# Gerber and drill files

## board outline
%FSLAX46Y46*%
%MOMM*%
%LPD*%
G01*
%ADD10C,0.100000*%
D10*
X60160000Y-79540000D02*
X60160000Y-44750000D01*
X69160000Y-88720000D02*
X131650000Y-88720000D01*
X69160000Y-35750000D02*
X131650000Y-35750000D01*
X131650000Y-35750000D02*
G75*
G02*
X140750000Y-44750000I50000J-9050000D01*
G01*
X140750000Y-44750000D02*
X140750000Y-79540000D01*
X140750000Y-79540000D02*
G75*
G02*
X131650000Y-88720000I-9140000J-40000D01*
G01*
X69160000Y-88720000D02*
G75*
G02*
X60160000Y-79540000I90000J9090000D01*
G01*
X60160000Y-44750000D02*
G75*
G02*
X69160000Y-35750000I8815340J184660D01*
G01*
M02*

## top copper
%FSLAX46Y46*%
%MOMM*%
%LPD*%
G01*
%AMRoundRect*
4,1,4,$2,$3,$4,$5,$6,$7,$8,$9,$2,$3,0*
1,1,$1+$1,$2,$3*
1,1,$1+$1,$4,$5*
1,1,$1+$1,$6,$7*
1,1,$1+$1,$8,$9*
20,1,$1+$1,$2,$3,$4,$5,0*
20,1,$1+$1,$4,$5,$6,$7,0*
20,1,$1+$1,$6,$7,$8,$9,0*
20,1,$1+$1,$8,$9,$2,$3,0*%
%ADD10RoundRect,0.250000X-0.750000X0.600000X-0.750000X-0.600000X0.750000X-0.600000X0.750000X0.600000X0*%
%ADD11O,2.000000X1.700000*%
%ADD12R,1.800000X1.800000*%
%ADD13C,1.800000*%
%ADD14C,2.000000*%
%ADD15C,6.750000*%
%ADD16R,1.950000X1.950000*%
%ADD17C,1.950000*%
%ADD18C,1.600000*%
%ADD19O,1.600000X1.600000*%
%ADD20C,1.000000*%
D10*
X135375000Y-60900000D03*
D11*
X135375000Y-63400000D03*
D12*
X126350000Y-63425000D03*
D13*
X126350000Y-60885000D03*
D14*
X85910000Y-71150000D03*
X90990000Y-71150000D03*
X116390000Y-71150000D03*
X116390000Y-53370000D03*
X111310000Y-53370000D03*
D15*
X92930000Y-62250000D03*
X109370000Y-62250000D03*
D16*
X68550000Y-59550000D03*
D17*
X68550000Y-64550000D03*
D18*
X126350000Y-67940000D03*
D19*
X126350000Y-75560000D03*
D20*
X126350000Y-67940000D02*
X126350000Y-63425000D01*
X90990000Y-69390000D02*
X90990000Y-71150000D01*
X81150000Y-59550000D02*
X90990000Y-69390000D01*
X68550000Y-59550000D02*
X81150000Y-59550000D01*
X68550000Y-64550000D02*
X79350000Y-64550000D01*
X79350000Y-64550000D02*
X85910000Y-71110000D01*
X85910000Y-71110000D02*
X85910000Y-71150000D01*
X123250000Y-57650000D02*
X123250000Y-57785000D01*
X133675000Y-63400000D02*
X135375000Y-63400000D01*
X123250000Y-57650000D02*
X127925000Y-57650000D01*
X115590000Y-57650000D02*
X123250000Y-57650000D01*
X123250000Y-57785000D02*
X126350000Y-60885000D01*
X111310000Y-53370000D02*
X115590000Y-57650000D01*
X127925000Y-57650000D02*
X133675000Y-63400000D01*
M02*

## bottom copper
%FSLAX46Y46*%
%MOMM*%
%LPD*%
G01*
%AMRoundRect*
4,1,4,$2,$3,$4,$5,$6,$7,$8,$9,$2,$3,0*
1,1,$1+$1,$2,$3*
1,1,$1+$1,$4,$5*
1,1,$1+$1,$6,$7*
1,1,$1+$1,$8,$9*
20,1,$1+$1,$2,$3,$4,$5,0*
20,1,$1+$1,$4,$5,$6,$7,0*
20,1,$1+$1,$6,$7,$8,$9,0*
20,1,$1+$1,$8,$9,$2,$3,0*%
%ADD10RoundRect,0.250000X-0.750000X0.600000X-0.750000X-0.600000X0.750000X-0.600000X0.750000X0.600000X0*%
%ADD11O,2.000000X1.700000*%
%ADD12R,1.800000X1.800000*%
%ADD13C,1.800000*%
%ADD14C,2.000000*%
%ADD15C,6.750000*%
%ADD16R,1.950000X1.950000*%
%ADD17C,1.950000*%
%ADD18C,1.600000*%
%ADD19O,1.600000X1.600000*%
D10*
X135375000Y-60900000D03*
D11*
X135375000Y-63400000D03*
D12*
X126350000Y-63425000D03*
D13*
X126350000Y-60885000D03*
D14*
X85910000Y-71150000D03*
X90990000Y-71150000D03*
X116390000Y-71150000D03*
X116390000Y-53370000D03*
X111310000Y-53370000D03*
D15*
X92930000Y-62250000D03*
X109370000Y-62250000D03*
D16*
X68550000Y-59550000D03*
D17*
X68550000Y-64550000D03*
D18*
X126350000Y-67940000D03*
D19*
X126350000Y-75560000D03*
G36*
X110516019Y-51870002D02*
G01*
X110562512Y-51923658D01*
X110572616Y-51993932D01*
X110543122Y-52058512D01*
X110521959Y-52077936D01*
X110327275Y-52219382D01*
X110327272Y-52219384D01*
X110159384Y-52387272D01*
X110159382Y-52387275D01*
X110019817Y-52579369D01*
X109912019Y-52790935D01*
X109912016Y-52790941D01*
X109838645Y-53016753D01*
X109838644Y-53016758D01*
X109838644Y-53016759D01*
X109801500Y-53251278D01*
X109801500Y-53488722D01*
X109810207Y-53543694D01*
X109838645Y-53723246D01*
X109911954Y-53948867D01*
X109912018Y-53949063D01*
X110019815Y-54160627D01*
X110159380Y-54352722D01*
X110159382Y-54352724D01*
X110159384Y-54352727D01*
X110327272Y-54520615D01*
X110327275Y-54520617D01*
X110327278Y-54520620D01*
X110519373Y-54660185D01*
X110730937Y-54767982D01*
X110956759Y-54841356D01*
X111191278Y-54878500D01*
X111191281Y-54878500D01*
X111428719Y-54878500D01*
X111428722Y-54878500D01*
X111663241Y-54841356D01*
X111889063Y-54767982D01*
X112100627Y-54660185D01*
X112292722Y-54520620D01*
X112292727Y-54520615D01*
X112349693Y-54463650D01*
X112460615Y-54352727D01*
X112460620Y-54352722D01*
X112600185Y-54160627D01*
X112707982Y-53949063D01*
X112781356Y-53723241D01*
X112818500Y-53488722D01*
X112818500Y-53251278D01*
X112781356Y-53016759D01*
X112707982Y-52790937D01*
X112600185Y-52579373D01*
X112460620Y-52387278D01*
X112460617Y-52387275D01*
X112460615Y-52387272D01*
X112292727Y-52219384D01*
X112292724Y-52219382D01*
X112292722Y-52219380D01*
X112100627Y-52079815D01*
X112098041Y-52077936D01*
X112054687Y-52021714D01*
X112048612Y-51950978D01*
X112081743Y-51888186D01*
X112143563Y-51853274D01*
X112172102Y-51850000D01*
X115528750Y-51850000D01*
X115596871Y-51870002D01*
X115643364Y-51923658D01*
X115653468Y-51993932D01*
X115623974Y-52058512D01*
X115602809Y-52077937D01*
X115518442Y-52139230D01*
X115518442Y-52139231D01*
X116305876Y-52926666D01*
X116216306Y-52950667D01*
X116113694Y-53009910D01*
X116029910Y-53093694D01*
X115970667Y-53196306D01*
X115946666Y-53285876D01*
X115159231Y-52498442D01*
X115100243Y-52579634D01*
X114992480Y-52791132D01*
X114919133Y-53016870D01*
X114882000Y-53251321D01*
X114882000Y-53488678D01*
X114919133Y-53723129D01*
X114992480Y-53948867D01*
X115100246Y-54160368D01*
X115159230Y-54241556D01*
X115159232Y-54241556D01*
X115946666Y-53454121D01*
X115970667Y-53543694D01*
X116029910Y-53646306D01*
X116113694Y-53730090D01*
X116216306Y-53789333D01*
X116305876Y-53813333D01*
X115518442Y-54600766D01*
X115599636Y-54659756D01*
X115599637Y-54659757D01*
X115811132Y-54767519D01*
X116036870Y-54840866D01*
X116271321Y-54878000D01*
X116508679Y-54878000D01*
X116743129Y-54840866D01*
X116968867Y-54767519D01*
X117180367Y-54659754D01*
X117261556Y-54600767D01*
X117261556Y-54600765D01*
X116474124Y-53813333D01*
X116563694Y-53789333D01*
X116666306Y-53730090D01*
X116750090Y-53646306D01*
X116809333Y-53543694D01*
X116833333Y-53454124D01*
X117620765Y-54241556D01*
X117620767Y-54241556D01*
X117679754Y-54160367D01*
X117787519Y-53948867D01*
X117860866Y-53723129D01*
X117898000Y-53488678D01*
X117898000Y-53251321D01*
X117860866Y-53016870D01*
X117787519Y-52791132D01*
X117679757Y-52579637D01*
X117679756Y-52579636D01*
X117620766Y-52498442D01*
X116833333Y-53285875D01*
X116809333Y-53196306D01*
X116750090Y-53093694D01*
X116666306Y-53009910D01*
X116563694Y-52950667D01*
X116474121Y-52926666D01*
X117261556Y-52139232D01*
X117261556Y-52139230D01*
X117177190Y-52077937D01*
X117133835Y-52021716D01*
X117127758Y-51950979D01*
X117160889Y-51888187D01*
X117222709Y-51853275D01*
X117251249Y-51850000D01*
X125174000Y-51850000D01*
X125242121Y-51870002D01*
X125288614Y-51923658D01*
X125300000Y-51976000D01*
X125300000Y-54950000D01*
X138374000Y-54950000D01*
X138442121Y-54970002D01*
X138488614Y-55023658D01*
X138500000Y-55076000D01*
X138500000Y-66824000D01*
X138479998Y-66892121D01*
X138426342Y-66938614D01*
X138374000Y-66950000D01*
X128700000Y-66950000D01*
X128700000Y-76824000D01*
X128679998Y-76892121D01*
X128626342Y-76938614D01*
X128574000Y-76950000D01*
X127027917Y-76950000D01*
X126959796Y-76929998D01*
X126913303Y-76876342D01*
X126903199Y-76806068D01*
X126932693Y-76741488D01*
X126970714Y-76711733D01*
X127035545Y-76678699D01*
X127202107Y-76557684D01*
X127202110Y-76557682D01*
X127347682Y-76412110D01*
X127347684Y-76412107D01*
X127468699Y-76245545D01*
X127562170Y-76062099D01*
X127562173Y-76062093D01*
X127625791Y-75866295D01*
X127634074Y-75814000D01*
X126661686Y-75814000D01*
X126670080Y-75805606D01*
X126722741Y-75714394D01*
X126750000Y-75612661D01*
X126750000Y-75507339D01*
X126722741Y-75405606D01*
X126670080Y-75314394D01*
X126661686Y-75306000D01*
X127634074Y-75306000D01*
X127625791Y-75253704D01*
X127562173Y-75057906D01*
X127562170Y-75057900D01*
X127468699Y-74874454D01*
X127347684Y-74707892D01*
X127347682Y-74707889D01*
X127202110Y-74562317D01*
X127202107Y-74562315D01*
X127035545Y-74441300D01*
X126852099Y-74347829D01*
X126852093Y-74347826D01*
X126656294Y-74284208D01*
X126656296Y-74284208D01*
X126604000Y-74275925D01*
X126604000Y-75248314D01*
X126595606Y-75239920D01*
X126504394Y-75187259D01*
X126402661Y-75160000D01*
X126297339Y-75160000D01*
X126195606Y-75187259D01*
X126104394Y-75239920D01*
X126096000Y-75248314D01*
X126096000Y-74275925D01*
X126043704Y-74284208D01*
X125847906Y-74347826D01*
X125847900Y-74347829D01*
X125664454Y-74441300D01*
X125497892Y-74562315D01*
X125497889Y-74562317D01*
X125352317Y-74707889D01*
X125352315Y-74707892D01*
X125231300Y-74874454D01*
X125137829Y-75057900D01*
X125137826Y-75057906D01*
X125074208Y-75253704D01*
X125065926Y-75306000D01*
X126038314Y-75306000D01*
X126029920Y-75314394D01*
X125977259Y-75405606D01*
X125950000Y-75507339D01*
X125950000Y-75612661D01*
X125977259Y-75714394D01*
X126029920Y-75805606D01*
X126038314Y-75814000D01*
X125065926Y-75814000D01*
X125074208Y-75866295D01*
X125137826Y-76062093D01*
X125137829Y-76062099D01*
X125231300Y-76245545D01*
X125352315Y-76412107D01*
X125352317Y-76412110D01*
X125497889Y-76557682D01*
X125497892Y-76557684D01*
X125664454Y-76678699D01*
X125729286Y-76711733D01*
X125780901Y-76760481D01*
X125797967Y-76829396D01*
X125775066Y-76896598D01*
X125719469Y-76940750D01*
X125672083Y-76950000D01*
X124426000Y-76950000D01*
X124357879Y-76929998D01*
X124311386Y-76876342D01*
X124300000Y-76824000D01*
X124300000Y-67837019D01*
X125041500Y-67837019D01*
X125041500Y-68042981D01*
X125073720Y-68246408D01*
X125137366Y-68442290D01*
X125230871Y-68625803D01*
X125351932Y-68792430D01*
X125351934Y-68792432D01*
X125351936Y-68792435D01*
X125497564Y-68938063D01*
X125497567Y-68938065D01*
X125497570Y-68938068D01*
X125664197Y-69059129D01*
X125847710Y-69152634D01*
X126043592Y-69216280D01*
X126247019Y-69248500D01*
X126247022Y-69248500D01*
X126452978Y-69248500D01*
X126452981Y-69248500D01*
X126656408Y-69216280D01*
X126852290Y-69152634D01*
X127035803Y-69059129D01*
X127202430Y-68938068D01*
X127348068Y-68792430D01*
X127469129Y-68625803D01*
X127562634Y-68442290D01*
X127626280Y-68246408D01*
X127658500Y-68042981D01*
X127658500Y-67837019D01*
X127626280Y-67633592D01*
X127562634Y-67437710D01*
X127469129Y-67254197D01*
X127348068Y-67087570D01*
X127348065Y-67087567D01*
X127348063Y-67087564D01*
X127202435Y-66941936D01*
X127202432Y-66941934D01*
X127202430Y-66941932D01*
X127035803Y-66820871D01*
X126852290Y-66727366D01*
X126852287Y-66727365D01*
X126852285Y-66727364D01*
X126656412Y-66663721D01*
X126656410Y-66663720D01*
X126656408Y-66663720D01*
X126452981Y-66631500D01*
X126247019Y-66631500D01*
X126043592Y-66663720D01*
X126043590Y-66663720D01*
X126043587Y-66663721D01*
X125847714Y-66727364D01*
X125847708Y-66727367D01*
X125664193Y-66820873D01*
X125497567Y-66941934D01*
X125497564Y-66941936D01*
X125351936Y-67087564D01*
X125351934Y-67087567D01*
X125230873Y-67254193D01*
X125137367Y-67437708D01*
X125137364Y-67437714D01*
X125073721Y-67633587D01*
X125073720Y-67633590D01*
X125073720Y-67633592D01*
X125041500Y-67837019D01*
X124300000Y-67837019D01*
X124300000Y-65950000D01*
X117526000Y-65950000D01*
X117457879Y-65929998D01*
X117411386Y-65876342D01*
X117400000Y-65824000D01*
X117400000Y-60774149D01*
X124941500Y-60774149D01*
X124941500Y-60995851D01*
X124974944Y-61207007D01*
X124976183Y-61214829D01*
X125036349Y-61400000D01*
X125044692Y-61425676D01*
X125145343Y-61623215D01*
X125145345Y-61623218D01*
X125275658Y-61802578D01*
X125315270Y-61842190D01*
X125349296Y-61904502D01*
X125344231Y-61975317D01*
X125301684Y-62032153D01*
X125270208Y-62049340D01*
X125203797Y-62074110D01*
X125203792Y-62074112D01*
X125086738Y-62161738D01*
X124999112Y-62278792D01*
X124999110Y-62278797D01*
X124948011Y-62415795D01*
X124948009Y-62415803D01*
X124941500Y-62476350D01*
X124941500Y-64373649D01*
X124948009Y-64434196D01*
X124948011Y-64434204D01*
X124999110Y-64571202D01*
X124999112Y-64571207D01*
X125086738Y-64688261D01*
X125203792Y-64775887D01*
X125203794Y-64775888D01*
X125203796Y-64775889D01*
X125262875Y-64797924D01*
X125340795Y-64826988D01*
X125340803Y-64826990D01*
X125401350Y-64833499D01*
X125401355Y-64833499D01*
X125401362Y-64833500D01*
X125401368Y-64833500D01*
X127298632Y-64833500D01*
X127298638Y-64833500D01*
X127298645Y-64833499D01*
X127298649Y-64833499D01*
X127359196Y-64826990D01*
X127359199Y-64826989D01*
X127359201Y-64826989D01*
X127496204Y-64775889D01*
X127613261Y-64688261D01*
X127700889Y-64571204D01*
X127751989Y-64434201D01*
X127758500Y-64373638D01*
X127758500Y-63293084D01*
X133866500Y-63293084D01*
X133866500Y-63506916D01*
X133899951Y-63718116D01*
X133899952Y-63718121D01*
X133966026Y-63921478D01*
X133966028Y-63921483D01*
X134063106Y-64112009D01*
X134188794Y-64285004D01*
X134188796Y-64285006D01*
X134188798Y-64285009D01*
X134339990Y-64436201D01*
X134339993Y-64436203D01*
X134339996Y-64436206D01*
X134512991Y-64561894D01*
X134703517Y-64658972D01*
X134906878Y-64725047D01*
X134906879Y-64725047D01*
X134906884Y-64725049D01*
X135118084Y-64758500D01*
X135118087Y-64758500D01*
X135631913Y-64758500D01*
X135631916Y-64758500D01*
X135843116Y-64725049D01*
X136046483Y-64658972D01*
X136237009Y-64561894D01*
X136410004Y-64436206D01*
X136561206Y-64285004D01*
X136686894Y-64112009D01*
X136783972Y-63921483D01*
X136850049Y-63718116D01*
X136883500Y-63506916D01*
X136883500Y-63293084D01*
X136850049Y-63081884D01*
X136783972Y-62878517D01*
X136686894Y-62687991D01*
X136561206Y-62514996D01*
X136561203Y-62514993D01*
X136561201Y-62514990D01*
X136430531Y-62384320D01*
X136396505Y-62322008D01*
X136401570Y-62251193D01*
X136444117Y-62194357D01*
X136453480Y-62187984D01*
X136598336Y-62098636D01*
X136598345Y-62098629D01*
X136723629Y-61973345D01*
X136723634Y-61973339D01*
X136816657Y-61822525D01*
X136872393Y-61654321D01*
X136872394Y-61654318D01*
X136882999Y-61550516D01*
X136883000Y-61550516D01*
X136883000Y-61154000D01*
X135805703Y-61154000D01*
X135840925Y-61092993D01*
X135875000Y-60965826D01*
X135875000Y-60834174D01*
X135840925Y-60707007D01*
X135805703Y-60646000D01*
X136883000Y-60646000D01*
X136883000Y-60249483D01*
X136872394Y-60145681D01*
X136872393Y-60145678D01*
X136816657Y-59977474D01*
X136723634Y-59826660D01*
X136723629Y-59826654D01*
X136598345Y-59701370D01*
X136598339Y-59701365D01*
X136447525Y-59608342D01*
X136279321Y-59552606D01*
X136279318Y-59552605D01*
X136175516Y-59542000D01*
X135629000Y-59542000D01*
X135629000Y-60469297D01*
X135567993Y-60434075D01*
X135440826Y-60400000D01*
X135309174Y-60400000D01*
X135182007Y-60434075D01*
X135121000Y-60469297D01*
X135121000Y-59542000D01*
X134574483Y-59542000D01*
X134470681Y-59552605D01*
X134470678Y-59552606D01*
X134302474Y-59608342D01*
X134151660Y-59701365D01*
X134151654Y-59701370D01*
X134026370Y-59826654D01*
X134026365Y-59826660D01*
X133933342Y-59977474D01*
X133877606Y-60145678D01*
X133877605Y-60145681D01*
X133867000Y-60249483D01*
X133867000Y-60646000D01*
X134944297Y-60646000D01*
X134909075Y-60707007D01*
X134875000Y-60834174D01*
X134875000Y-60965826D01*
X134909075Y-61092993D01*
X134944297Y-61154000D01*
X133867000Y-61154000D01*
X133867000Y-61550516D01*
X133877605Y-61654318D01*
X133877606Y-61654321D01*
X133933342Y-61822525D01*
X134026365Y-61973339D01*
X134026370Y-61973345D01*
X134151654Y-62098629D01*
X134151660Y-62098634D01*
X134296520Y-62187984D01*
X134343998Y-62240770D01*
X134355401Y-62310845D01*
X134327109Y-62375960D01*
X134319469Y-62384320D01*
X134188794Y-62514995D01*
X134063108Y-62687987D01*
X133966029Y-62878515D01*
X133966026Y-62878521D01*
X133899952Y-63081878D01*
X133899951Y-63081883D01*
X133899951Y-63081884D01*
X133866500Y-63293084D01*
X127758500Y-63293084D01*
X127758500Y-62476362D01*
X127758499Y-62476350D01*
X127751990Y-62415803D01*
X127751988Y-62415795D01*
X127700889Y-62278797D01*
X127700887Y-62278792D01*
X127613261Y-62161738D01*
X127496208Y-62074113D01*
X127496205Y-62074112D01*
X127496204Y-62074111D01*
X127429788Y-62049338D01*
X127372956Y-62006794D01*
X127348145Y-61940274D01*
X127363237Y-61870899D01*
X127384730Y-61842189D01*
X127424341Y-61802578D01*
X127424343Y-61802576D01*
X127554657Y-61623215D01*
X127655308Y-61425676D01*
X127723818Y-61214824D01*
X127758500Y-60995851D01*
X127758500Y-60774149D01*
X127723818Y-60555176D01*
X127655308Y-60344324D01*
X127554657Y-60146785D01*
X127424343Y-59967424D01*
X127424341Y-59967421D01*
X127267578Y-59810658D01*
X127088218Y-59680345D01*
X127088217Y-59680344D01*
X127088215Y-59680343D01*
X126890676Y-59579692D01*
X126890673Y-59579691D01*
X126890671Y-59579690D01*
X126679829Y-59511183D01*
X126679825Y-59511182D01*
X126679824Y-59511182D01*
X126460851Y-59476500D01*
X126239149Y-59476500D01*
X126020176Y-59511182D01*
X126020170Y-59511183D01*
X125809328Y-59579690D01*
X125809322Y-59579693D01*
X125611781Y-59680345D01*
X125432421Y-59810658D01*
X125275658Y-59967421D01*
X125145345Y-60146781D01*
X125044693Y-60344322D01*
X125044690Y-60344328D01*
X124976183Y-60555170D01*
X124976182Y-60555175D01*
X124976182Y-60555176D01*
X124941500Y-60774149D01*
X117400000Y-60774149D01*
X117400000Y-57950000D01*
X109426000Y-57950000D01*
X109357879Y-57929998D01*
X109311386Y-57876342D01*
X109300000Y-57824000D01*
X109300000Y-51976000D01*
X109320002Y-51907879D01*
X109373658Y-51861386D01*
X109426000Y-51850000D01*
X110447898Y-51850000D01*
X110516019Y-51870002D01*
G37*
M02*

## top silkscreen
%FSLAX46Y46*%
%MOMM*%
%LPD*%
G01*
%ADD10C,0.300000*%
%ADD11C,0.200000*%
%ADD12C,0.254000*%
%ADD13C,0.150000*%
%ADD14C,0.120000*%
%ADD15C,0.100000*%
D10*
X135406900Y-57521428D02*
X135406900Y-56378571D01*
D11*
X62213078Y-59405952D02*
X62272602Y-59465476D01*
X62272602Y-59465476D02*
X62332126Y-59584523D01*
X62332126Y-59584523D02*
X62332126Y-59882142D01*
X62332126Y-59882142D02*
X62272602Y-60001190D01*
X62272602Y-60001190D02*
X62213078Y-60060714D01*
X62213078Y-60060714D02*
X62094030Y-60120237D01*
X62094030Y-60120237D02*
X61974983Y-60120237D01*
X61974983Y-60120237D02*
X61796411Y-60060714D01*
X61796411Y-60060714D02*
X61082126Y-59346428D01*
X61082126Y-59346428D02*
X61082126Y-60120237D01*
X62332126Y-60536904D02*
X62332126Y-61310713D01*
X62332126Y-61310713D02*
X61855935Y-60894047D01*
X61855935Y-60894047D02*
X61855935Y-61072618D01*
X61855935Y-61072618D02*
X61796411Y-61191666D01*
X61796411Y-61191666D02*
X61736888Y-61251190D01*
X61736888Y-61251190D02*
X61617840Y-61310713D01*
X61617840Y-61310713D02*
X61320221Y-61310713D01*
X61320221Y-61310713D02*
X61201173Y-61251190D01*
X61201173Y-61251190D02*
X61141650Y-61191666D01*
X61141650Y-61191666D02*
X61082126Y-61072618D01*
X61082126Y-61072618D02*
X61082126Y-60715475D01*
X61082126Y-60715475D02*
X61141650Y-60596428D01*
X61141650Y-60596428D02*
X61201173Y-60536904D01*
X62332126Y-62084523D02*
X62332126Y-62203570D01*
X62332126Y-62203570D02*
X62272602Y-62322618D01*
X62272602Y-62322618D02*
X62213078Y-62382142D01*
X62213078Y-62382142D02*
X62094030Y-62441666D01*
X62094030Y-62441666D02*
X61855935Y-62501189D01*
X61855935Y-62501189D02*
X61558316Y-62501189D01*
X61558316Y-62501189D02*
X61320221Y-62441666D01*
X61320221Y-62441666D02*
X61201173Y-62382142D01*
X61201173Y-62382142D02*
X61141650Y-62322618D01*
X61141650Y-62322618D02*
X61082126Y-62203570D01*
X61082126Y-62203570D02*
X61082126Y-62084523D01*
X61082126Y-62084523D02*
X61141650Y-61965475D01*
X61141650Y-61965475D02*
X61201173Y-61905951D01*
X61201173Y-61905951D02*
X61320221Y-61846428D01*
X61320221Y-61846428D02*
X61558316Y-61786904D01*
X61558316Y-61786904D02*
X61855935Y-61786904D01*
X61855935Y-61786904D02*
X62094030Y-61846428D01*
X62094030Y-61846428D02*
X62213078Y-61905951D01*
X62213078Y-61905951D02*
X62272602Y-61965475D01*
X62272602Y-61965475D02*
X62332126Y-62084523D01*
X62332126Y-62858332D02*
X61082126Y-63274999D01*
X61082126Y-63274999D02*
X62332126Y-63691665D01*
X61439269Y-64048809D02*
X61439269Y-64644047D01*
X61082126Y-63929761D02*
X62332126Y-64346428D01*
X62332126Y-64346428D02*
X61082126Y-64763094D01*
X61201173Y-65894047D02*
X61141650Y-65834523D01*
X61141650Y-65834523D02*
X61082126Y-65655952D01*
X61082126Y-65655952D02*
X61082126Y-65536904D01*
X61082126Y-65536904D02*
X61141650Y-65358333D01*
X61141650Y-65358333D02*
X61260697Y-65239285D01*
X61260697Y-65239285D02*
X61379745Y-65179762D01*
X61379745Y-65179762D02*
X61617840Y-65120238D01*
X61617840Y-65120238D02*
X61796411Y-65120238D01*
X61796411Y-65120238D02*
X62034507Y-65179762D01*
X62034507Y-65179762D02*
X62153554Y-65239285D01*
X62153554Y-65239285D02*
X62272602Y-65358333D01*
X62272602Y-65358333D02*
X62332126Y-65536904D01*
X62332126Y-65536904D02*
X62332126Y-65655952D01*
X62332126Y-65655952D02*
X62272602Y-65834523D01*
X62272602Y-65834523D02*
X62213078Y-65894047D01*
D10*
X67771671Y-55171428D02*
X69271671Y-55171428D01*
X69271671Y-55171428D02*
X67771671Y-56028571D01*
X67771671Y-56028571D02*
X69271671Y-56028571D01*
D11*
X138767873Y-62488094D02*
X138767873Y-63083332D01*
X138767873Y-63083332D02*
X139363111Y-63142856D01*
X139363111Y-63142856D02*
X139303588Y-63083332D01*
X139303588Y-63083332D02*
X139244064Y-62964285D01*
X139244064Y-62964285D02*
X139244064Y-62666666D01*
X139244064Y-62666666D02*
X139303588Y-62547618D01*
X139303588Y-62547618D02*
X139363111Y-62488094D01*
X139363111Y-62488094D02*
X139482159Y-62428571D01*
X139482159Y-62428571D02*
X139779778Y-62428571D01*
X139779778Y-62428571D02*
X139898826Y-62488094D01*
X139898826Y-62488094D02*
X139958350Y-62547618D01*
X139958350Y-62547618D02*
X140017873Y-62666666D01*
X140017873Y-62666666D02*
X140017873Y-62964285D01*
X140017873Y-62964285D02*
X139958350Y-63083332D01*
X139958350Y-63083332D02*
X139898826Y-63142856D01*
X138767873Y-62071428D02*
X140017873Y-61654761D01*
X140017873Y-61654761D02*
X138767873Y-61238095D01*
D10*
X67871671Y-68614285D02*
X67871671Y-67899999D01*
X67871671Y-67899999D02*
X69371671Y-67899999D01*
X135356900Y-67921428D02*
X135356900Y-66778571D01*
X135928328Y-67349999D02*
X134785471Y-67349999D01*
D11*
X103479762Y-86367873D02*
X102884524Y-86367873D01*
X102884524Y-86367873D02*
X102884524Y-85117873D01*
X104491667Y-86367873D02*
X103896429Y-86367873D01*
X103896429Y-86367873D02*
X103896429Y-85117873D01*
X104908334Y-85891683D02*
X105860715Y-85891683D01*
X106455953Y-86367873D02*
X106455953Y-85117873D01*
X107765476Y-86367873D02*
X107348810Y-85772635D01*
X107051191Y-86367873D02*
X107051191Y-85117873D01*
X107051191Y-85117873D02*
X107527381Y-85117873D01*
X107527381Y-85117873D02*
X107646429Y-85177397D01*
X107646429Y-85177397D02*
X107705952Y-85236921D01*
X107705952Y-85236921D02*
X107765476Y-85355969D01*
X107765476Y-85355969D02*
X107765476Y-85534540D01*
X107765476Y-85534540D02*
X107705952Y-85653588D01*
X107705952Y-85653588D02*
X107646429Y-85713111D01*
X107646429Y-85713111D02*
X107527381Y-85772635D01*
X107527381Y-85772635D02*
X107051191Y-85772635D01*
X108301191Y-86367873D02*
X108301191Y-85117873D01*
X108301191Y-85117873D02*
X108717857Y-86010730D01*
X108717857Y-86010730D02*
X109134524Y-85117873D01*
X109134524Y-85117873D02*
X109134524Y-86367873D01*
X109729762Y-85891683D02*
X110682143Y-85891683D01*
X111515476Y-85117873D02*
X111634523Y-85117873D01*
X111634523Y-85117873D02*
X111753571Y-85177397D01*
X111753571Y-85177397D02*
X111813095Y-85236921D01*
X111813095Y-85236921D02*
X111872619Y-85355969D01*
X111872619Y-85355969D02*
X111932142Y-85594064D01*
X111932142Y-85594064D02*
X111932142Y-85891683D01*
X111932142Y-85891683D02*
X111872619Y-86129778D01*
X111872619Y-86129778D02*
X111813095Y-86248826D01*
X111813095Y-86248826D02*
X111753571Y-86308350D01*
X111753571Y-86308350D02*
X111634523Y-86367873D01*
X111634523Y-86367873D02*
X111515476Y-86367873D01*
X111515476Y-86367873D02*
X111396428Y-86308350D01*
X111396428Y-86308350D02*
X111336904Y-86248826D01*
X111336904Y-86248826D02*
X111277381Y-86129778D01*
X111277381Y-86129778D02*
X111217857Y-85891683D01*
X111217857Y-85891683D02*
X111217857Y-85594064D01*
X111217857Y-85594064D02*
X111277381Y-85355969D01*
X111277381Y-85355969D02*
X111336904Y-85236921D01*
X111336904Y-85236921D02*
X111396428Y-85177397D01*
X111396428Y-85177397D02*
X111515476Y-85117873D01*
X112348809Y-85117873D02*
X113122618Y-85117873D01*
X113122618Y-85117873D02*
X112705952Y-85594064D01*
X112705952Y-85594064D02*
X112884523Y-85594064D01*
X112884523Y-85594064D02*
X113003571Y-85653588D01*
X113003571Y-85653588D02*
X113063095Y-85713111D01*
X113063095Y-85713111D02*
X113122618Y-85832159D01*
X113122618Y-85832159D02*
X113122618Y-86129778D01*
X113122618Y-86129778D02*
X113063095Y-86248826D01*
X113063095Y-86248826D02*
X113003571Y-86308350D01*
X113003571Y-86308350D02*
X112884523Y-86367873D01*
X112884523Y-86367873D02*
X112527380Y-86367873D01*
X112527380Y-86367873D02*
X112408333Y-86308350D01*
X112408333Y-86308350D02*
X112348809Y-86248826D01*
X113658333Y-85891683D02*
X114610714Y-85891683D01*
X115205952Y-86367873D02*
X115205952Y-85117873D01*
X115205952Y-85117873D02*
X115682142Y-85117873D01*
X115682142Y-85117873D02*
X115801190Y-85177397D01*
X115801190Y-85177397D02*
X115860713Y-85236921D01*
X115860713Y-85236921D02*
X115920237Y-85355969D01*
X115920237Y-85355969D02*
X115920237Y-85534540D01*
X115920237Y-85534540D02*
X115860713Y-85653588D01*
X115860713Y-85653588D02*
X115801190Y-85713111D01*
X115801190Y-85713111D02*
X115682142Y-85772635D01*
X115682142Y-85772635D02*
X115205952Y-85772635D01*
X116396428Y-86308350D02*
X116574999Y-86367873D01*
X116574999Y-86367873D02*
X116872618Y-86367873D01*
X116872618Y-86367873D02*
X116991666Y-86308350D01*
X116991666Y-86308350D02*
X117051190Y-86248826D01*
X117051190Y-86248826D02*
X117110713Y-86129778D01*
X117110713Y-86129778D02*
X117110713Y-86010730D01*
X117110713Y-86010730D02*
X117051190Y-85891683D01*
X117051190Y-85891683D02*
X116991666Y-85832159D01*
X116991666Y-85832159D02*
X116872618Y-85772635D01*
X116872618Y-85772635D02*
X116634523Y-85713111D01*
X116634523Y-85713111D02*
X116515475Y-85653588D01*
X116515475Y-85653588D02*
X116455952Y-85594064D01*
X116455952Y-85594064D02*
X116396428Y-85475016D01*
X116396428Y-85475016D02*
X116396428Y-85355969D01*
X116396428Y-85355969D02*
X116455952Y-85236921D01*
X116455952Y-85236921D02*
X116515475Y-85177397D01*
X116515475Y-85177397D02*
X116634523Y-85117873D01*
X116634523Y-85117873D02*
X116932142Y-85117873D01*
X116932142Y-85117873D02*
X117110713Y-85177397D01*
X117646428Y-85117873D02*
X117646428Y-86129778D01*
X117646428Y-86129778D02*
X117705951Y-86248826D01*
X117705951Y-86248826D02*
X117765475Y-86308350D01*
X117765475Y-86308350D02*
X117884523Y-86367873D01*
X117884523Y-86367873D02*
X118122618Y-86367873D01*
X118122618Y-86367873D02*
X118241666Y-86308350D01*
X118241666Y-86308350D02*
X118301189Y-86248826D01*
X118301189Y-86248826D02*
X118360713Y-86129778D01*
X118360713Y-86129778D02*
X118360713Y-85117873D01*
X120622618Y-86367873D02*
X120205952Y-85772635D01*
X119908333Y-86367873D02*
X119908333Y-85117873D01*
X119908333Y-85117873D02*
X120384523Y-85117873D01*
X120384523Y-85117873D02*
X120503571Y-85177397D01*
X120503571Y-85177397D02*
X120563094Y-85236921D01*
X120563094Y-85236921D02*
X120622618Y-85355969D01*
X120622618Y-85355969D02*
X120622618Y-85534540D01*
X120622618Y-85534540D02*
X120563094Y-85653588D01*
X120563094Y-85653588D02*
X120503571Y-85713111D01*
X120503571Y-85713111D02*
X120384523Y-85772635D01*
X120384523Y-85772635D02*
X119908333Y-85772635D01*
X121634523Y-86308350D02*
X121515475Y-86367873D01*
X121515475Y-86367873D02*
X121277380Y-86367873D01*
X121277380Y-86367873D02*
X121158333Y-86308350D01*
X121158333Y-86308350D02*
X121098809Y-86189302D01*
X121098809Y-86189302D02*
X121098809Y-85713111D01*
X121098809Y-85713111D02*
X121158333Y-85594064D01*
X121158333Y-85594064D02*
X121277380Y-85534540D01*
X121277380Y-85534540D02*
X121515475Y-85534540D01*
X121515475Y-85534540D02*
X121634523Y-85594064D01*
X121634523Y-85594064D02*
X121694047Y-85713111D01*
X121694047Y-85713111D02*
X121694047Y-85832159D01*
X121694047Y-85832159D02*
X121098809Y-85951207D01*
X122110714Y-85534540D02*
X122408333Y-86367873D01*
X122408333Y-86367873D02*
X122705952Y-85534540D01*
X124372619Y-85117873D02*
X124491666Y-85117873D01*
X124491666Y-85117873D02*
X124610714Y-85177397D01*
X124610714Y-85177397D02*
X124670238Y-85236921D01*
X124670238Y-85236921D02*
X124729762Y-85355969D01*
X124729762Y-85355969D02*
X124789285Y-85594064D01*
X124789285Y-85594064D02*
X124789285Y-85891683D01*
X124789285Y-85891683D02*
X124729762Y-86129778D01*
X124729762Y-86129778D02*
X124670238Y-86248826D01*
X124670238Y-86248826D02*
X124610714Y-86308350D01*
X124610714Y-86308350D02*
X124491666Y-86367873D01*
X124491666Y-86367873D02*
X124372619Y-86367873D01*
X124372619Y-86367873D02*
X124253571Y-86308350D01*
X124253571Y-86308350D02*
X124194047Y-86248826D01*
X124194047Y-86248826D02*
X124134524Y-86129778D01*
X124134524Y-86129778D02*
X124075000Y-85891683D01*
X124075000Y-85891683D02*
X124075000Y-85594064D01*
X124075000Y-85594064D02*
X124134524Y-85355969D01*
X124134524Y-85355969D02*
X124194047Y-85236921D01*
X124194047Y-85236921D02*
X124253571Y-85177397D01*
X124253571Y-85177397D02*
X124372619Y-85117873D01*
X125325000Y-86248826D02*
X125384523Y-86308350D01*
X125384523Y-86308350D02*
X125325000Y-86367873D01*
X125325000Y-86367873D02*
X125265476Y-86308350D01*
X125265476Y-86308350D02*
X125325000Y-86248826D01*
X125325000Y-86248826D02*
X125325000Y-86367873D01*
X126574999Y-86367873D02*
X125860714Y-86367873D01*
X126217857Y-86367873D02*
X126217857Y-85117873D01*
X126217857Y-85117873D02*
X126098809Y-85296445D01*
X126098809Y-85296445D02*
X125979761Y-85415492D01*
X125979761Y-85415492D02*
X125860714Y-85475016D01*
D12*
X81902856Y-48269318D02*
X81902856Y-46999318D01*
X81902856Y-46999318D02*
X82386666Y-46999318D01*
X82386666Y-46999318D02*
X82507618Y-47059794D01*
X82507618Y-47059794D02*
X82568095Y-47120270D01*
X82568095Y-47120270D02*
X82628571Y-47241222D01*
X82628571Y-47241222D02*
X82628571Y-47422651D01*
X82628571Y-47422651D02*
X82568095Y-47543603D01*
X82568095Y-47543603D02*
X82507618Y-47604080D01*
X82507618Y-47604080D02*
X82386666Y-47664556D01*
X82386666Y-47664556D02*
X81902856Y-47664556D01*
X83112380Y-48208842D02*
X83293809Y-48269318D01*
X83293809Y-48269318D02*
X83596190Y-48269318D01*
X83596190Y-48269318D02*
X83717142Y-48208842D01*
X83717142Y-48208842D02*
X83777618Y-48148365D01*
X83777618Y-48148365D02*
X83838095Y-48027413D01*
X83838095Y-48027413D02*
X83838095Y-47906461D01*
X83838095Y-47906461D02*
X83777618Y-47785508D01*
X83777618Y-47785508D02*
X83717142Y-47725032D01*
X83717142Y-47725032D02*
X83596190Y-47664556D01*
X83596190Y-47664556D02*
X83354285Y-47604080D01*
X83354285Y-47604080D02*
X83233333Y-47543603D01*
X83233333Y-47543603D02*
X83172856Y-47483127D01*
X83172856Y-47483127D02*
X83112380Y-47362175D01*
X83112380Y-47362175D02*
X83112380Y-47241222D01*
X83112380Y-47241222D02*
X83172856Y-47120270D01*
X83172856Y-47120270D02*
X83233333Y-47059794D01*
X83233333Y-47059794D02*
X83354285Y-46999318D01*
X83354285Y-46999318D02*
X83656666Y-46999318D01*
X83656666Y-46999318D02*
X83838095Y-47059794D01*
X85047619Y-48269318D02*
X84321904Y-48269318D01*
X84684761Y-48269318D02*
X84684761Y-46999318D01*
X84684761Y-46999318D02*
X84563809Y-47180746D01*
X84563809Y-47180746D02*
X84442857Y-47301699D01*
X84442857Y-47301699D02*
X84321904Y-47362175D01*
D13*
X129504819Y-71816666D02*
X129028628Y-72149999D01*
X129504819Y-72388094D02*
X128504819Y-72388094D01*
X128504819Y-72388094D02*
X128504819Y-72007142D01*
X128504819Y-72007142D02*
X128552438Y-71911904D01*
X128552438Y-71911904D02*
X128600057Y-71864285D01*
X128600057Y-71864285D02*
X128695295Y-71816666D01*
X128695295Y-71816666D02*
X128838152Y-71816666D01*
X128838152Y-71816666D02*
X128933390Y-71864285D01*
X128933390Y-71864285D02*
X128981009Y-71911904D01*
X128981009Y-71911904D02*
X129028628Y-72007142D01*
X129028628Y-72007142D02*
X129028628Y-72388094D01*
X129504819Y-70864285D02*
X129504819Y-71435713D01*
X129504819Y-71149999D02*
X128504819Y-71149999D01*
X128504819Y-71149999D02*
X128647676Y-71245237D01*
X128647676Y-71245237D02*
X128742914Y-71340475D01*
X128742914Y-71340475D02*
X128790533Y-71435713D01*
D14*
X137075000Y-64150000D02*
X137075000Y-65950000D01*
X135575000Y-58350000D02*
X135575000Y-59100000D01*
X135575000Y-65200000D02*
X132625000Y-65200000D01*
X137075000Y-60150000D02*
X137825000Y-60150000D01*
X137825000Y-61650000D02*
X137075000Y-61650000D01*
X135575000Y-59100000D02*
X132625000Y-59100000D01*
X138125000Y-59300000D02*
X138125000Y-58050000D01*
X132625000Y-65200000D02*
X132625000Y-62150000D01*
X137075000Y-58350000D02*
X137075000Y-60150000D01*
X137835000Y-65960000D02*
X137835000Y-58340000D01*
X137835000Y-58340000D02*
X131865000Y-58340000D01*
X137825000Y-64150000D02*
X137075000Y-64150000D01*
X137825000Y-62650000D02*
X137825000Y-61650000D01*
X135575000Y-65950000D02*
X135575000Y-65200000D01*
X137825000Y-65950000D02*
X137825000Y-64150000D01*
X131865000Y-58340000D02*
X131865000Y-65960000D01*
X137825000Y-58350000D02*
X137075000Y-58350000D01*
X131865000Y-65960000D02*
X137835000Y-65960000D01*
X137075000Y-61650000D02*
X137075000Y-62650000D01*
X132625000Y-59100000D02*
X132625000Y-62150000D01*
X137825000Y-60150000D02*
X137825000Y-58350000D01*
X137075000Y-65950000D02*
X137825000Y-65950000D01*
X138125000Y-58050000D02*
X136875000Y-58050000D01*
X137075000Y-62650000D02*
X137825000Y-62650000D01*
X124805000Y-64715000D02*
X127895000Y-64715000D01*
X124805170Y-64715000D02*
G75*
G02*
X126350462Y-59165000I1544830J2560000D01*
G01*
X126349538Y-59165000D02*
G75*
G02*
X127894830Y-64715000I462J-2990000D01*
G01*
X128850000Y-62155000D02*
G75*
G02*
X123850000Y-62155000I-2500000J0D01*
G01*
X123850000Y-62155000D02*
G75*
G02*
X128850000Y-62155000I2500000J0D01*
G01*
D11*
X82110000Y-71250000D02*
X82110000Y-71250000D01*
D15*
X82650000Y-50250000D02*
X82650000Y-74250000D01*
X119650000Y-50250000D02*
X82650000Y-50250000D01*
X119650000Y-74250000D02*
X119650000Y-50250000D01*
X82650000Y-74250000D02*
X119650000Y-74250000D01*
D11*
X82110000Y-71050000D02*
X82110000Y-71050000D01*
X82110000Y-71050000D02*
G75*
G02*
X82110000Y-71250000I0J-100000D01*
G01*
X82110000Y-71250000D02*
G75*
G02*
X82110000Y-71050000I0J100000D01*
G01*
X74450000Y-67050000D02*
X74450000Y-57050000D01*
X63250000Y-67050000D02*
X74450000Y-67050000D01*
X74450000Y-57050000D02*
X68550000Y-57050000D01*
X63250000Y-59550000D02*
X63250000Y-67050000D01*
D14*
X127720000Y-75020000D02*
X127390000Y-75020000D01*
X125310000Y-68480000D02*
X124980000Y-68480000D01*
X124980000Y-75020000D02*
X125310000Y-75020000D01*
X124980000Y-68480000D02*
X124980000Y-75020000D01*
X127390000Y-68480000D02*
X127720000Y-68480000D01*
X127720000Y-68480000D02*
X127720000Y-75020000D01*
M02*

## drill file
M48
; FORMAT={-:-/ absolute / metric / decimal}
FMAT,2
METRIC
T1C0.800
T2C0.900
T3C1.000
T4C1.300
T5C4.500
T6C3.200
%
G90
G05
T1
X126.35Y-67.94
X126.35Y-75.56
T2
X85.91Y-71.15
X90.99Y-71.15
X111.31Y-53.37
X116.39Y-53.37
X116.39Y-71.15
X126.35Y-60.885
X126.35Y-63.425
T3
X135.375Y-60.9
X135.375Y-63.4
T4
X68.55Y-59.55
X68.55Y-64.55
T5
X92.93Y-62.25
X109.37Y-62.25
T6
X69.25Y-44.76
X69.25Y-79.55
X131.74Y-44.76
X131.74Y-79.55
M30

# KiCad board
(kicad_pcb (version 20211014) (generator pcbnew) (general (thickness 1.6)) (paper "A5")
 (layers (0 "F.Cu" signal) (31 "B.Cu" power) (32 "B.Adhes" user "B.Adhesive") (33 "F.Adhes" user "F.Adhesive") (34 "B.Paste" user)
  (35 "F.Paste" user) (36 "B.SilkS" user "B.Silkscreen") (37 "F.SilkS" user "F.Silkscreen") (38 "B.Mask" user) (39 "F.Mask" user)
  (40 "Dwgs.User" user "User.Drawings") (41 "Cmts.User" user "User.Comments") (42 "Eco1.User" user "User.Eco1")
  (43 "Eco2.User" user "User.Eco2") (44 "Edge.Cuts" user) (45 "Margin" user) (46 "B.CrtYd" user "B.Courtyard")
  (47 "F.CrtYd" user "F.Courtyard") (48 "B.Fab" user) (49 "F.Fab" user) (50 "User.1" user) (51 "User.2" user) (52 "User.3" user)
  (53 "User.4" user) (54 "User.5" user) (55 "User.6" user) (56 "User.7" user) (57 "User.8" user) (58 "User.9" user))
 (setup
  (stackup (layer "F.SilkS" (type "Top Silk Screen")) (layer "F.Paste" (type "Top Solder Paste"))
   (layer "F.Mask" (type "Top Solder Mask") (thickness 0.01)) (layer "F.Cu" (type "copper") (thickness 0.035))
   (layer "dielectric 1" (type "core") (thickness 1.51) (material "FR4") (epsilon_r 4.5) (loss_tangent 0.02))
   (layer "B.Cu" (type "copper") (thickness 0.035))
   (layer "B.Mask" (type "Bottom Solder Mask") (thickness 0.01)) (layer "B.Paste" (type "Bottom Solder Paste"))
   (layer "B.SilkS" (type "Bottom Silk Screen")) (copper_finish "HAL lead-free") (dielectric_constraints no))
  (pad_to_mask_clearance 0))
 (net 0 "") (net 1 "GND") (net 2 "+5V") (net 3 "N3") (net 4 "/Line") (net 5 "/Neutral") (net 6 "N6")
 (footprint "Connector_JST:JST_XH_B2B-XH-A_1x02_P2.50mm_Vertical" (layer "F.Cu") (at 135.375 60.9 -90)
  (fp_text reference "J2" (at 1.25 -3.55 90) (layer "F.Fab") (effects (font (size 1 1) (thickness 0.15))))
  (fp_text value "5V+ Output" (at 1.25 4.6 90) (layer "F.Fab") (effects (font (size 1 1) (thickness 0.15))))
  (fp_line (start 3.25 -1.7) (end 5.05 -1.7) (layer "F.SilkS") (width 0.12))
  (fp_line (start -2.55 -0.2) (end -1.8 -0.2) (layer "F.SilkS") (width 0.12))
  (fp_line (start 4.3 -0.2) (end 4.3 2.75) (layer "F.SilkS") (width 0.12))
  (fp_line (start -0.75 -1.7) (end -0.75 -2.45) (layer "F.SilkS") (width 0.12))
  (fp_line (start 0.75 -2.45) (end 0.75 -1.7) (layer "F.SilkS") (width 0.12))
  (fp_line (start -1.8 -0.2) (end -1.8 2.75) (layer "F.SilkS") (width 0.12))
  (fp_line (start -1.6 -2.75) (end -2.85 -2.75) (layer "F.SilkS") (width 0.12))
  (fp_line (start 4.3 2.75) (end 1.25 2.75) (layer "F.SilkS") (width 0.12))
  (fp_line (start -2.55 -1.7) (end -0.75 -1.7) (layer "F.SilkS") (width 0.12))
  (fp_line (start 5.06 -2.46) (end -2.56 -2.46) (layer "F.SilkS") (width 0.12))
  (fp_line (start -2.56 -2.46) (end -2.56 3.51) (layer "F.SilkS") (width 0.12))
  (fp_line (start 3.25 -2.45) (end 3.25 -1.7) (layer "F.SilkS") (width 0.12))
  (fp_line (start 1.75 -2.45) (end 0.75 -2.45) (layer "F.SilkS") (width 0.12))
  (fp_line (start 5.05 -0.2) (end 4.3 -0.2) (layer "F.SilkS") (width 0.12))
  (fp_line (start 5.05 -2.45) (end 3.25 -2.45) (layer "F.SilkS") (width 0.12))
  (fp_line (start -2.56 3.51) (end 5.06 3.51) (layer "F.SilkS") (width 0.12))
  (fp_line (start -2.55 -2.45) (end -2.55 -1.7) (layer "F.SilkS") (width 0.12))
  (fp_line (start 5.06 3.51) (end 5.06 -2.46) (layer "F.SilkS") (width 0.12))
  (fp_line (start 0.75 -1.7) (end 1.75 -1.7) (layer "F.SilkS") (width 0.12))
  (fp_line (start -1.8 2.75) (end 1.25 2.75) (layer "F.SilkS") (width 0.12))
  (fp_line (start -0.75 -2.45) (end -2.55 -2.45) (layer "F.SilkS") (width 0.12))
  (fp_line (start 5.05 -1.7) (end 5.05 -2.45) (layer "F.SilkS") (width 0.12))
  (fp_line (start -2.85 -2.75) (end -2.85 -1.5) (layer "F.SilkS") (width 0.12))
  (fp_line (start 1.75 -1.7) (end 1.75 -2.45) (layer "F.SilkS") (width 0.12))
  (pad "1" thru_hole roundrect (at 0 0 270) (size 1.7 2) (drill 1) (layers *.Cu *.Mask) (roundrect_rratio 0.1470588235) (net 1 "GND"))
  (pad "2" thru_hole oval (at 2.5 0 270) (size 1.7 2) (drill 1) (layers *.Cu *.Mask) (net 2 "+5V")))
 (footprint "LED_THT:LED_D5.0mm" (layer "F.Cu") (at 126.35 63.425 90)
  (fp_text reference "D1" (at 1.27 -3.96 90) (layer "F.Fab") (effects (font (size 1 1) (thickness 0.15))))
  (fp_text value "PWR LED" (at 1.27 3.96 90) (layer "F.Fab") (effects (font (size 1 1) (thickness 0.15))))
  (fp_line (start -1.29 -1.545) (end -1.29 1.545) (layer "F.SilkS") (width 0.12))
  (fp_arc (start -1.29 -1.54483) (mid 2.072002 -2.880433) (end 4.26 0.000462) (layer "F.SilkS") (width 0.12))
  (fp_arc (start 4.26 -0.000462) (mid 2.072002 2.880433) (end -1.29 1.54483) (layer "F.SilkS") (width 0.12))
  (fp_circle (center 1.27 0) (end 3.77 0) (layer "F.SilkS") (width 0.12) (fill none))
  (pad "1" thru_hole rect (at 0 0 90) (size 1.8 1.8) (drill 0.9) (layers *.Cu *.Mask) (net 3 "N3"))
  (pad "2" thru_hole circle (at 2.54 0 90) (size 1.8 1.8) (drill 0.9) (layers *.Cu *.Mask) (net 2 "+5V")))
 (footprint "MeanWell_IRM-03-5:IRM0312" (layer "F.Cu") (at 85.91 71.15)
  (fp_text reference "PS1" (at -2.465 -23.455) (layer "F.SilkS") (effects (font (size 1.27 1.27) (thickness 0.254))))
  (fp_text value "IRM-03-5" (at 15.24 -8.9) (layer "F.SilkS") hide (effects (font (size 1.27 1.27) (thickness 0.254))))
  (fp_line (start -3.8 0.1) (end -3.8 0.1) (layer "F.SilkS") (width 0.2))
  (fp_line (start -3.26 -20.9) (end -3.26 3.1) (layer "F.SilkS") (width 0.1))
  (fp_line (start 33.74 -20.9) (end -3.26 -20.9) (layer "F.SilkS") (width 0.1))
  (fp_line (start 33.74 3.1) (end 33.74 -20.9) (layer "F.SilkS") (width 0.1))
  (fp_line (start -3.26 3.1) (end 33.74 3.1) (layer "F.SilkS") (width 0.1))
  (fp_line (start -3.8 -0.1) (end -3.8 -0.1) (layer "F.SilkS") (width 0.2))
  (fp_arc (start -3.8 -0.1) (mid -3.7 0) (end -3.8 0.1) (layer "F.SilkS") (width 0.2))
  (fp_arc (start -3.8 0.1) (mid -3.9 0) (end -3.8 -0.1) (layer "F.SilkS") (width 0.2))
  (pad "1" thru_hole circle (at 0 0) (size 2 2) (drill 0.9) (layers *.Cu *.Mask) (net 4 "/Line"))
  (pad "2" thru_hole circle (at 5.08 0) (size 2 2) (drill 0.9) (layers *.Cu *.Mask) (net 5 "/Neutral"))
  (pad "3" thru_hole circle (at 30.48 0) (size 2 2) (drill 0.9) (layers *.Cu *.Mask) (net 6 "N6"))
  (pad "4" thru_hole circle (at 30.48 -17.78) (size 2 2) (drill 0.9) (layers *.Cu *.Mask) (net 1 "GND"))
  (pad "5" thru_hole circle (at 25.4 -17.78) (size 2 2) (drill 0.9) (layers *.Cu *.Mask) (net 2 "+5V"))
  (pad "6" thru_hole circle (at 7.02 -8.9) (size 6.75 6.75) (drill 4.5) (layers *.Cu *.Mask))
  (pad "7" thru_hole circle (at 23.46 -8.9) (size 6.75 6.75) (drill 4.5) (layers *.Cu *.Mask)))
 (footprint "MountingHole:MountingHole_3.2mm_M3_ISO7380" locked (layer "F.Cu") (at 69.25 44.76)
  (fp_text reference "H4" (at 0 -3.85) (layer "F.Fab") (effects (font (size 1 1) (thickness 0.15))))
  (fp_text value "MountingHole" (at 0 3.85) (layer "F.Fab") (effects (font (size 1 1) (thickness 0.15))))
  (pad "" np_thru_hole circle locked (at 0 0) (size 3.2 3.2) (drill 3.2) (layers F&B.Cu *.Mask)))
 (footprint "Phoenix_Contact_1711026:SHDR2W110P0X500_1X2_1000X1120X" (layer "F.Cu") (at 68.55 59.55 -90)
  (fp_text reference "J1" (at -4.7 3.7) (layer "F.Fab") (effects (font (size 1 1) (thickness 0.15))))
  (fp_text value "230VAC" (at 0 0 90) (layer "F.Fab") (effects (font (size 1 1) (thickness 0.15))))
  (fp_line (start 7.5 -5.9) (end -2.5 -5.9) (layer "F.SilkS") (width 0.2))
  (fp_line (start 7.5 5.3) (end 7.5 -5.9) (layer "F.SilkS") (width 0.2))
  (fp_line (start -2.5 -5.9) (end -2.5 0) (layer "F.SilkS") (width 0.2))
  (fp_line (start 0 5.3) (end 7.5 5.3) (layer "F.SilkS") (width 0.2))
  (pad "1" thru_hole rect (at 0 0 270) (size 1.95 1.95) (drill 1.3) (layers *.Cu *.Mask) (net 5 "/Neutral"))
  (pad "2" thru_hole circle (at 5 0 270) (size 1.95 1.95) (drill 1.3) (layers *.Cu *.Mask) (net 4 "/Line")))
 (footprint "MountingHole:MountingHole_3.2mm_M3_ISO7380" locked (layer "F.Cu") (at 131.74 44.76)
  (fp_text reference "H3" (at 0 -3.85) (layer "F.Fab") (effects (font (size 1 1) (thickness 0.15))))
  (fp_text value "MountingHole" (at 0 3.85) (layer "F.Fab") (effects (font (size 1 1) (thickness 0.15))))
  (pad "" np_thru_hole circle locked (at 0 0) (size 3.2 3.2) (drill 3.2) (layers *.Cu *.Mask)))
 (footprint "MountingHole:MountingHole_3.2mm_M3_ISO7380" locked (layer "F.Cu") (at 131.74 79.55)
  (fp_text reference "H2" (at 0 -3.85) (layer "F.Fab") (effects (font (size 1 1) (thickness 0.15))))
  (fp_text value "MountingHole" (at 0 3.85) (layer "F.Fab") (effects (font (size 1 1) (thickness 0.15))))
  (pad "" np_thru_hole circle locked (at 0 0) (size 3.2 3.2) (drill 3.2) (layers *.Cu *.Mask)))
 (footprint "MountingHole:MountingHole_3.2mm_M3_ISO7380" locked (layer "F.Cu") (at 69.25 79.55)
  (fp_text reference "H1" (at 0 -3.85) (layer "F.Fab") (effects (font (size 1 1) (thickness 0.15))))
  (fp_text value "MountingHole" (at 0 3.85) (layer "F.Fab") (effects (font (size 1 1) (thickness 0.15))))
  (pad "" np_thru_hole circle locked (at 0 0) (size 3.2 3.2) (drill 3.2) (layers *.Cu *.Mask)))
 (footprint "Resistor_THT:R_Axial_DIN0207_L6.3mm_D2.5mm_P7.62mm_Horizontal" (layer "F.Cu") (at 126.35 67.94 -90)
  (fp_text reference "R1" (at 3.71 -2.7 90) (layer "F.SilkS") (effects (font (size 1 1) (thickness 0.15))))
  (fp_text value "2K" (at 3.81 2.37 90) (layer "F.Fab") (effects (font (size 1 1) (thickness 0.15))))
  (fp_line (start 7.08 -1.37) (end 7.08 -1.04) (layer "F.SilkS") (width 0.12))
  (fp_line (start 0.54 1.04) (end 0.54 1.37) (layer "F.SilkS") (width 0.12))
  (fp_line (start 7.08 1.37) (end 7.08 1.04) (layer "F.SilkS") (width 0.12))
  (fp_line (start 0.54 1.37) (end 7.08 1.37) (layer "F.SilkS") (width 0.12))
  (fp_line (start 0.54 -1.04) (end 0.54 -1.37) (layer "F.SilkS") (width 0.12))
  (fp_line (start 0.54 -1.37) (end 7.08 -1.37) (layer "F.SilkS") (width 0.12))
  (pad "1" thru_hole circle (at 0 0 270) (size 1.6 1.6) (drill 0.8) (layers *.Cu *.Mask) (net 3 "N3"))
  (pad "2" thru_hole oval (at 7.62 0 270) (size 1.6 1.6) (drill 0.8) (layers *.Cu *.Mask) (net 1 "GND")))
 (gr_line (start 60.16 79.54) (end 60.16 44.75) (layer "Edge.Cuts") (width 0.1))
 (gr_line (start 69.16 88.72) (end 131.65 88.72) (layer "Edge.Cuts") (width 0.1))
 (gr_line (start 69.16 35.75) (end 131.65 35.75) (layer "Edge.Cuts") (width 0.1))
 (gr_arc (start 131.65 35.75) (mid 138.063961 38.365328) (end 140.75 44.75) (layer "Edge.Cuts") (width 0.1))
 (gr_line (start 140.75 44.75) (end 140.75 79.54) (layer "Edge.Cuts") (width 0.1))
 (gr_arc (start 140.75 79.54) (mid 138.10124 86.014672) (end 131.65 88.72) (layer "Edge.Cuts") (width 0.1))
 (gr_arc (start 69.16 88.72) (mid 62.75876 85.993961) (end 60.16 79.54) (layer "Edge.Cuts") (width 0.1))
 (gr_arc (start 60.16 44.75) (mid 62.740586 38.330586) (end 69.16 35.75) (layer "Edge.Cuts") (width 0.1))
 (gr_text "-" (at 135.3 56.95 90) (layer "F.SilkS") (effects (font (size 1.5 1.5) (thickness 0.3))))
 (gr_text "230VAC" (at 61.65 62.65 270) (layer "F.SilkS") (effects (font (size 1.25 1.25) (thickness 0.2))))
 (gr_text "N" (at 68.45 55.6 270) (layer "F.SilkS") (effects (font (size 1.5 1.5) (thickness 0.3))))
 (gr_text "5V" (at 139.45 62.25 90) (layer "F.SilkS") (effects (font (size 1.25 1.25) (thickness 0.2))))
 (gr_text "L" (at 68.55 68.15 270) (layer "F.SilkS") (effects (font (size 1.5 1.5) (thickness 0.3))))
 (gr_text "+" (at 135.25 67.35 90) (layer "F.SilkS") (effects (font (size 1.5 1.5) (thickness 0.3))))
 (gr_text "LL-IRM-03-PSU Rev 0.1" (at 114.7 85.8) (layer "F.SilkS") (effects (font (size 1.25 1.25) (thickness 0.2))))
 (segment (start 126.35 67.94) (end 126.35 63.425) (width 1) (layer "F.Cu") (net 3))
 (segment (start 90.99 69.39) (end 90.99 71.15) (width 1) (layer "F.Cu") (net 5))
 (segment (start 81.15 59.55) (end 90.99 69.39) (width 1) (layer "F.Cu") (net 5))
 (segment (start 68.55 59.55) (end 81.15 59.55) (width 1) (layer "F.Cu") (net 5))
 (segment (start 68.55 64.55) (end 79.35 64.55) (width 1) (layer "F.Cu") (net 4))
 (segment (start 79.35 64.55) (end 85.91 71.11) (width 1) (layer "F.Cu") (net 4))
 (segment (start 85.91 71.11) (end 85.91 71.15) (width 1) (layer "F.Cu") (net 4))
 (segment (start 123.25 57.65) (end 123.25 57.785) (width 1) (layer "F.Cu") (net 2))
 (segment (start 133.675 63.4) (end 135.375 63.4) (width 1) (layer "F.Cu") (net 2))
 (segment (start 123.25 57.65) (end 127.925 57.65) (width 1) (layer "F.Cu") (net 2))
 (segment (start 115.59 57.65) (end 123.25 57.65) (width 1) (layer "F.Cu") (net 2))
 (segment (start 123.25 57.785) (end 126.35 60.885) (width 1) (layer "F.Cu") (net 2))
 (segment (start 111.31 53.37) (end 115.59 57.65) (width 1) (layer "F.Cu") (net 2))
 (segment (start 127.925 57.65) (end 133.675 63.4) (width 1) (layer "F.Cu") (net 2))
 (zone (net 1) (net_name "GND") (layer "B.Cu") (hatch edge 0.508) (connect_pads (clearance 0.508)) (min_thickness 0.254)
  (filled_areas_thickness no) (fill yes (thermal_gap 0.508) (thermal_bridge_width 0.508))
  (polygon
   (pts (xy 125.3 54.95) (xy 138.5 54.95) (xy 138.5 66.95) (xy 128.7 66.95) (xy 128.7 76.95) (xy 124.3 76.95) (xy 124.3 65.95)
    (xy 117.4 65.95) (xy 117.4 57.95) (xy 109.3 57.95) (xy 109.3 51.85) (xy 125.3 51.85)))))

